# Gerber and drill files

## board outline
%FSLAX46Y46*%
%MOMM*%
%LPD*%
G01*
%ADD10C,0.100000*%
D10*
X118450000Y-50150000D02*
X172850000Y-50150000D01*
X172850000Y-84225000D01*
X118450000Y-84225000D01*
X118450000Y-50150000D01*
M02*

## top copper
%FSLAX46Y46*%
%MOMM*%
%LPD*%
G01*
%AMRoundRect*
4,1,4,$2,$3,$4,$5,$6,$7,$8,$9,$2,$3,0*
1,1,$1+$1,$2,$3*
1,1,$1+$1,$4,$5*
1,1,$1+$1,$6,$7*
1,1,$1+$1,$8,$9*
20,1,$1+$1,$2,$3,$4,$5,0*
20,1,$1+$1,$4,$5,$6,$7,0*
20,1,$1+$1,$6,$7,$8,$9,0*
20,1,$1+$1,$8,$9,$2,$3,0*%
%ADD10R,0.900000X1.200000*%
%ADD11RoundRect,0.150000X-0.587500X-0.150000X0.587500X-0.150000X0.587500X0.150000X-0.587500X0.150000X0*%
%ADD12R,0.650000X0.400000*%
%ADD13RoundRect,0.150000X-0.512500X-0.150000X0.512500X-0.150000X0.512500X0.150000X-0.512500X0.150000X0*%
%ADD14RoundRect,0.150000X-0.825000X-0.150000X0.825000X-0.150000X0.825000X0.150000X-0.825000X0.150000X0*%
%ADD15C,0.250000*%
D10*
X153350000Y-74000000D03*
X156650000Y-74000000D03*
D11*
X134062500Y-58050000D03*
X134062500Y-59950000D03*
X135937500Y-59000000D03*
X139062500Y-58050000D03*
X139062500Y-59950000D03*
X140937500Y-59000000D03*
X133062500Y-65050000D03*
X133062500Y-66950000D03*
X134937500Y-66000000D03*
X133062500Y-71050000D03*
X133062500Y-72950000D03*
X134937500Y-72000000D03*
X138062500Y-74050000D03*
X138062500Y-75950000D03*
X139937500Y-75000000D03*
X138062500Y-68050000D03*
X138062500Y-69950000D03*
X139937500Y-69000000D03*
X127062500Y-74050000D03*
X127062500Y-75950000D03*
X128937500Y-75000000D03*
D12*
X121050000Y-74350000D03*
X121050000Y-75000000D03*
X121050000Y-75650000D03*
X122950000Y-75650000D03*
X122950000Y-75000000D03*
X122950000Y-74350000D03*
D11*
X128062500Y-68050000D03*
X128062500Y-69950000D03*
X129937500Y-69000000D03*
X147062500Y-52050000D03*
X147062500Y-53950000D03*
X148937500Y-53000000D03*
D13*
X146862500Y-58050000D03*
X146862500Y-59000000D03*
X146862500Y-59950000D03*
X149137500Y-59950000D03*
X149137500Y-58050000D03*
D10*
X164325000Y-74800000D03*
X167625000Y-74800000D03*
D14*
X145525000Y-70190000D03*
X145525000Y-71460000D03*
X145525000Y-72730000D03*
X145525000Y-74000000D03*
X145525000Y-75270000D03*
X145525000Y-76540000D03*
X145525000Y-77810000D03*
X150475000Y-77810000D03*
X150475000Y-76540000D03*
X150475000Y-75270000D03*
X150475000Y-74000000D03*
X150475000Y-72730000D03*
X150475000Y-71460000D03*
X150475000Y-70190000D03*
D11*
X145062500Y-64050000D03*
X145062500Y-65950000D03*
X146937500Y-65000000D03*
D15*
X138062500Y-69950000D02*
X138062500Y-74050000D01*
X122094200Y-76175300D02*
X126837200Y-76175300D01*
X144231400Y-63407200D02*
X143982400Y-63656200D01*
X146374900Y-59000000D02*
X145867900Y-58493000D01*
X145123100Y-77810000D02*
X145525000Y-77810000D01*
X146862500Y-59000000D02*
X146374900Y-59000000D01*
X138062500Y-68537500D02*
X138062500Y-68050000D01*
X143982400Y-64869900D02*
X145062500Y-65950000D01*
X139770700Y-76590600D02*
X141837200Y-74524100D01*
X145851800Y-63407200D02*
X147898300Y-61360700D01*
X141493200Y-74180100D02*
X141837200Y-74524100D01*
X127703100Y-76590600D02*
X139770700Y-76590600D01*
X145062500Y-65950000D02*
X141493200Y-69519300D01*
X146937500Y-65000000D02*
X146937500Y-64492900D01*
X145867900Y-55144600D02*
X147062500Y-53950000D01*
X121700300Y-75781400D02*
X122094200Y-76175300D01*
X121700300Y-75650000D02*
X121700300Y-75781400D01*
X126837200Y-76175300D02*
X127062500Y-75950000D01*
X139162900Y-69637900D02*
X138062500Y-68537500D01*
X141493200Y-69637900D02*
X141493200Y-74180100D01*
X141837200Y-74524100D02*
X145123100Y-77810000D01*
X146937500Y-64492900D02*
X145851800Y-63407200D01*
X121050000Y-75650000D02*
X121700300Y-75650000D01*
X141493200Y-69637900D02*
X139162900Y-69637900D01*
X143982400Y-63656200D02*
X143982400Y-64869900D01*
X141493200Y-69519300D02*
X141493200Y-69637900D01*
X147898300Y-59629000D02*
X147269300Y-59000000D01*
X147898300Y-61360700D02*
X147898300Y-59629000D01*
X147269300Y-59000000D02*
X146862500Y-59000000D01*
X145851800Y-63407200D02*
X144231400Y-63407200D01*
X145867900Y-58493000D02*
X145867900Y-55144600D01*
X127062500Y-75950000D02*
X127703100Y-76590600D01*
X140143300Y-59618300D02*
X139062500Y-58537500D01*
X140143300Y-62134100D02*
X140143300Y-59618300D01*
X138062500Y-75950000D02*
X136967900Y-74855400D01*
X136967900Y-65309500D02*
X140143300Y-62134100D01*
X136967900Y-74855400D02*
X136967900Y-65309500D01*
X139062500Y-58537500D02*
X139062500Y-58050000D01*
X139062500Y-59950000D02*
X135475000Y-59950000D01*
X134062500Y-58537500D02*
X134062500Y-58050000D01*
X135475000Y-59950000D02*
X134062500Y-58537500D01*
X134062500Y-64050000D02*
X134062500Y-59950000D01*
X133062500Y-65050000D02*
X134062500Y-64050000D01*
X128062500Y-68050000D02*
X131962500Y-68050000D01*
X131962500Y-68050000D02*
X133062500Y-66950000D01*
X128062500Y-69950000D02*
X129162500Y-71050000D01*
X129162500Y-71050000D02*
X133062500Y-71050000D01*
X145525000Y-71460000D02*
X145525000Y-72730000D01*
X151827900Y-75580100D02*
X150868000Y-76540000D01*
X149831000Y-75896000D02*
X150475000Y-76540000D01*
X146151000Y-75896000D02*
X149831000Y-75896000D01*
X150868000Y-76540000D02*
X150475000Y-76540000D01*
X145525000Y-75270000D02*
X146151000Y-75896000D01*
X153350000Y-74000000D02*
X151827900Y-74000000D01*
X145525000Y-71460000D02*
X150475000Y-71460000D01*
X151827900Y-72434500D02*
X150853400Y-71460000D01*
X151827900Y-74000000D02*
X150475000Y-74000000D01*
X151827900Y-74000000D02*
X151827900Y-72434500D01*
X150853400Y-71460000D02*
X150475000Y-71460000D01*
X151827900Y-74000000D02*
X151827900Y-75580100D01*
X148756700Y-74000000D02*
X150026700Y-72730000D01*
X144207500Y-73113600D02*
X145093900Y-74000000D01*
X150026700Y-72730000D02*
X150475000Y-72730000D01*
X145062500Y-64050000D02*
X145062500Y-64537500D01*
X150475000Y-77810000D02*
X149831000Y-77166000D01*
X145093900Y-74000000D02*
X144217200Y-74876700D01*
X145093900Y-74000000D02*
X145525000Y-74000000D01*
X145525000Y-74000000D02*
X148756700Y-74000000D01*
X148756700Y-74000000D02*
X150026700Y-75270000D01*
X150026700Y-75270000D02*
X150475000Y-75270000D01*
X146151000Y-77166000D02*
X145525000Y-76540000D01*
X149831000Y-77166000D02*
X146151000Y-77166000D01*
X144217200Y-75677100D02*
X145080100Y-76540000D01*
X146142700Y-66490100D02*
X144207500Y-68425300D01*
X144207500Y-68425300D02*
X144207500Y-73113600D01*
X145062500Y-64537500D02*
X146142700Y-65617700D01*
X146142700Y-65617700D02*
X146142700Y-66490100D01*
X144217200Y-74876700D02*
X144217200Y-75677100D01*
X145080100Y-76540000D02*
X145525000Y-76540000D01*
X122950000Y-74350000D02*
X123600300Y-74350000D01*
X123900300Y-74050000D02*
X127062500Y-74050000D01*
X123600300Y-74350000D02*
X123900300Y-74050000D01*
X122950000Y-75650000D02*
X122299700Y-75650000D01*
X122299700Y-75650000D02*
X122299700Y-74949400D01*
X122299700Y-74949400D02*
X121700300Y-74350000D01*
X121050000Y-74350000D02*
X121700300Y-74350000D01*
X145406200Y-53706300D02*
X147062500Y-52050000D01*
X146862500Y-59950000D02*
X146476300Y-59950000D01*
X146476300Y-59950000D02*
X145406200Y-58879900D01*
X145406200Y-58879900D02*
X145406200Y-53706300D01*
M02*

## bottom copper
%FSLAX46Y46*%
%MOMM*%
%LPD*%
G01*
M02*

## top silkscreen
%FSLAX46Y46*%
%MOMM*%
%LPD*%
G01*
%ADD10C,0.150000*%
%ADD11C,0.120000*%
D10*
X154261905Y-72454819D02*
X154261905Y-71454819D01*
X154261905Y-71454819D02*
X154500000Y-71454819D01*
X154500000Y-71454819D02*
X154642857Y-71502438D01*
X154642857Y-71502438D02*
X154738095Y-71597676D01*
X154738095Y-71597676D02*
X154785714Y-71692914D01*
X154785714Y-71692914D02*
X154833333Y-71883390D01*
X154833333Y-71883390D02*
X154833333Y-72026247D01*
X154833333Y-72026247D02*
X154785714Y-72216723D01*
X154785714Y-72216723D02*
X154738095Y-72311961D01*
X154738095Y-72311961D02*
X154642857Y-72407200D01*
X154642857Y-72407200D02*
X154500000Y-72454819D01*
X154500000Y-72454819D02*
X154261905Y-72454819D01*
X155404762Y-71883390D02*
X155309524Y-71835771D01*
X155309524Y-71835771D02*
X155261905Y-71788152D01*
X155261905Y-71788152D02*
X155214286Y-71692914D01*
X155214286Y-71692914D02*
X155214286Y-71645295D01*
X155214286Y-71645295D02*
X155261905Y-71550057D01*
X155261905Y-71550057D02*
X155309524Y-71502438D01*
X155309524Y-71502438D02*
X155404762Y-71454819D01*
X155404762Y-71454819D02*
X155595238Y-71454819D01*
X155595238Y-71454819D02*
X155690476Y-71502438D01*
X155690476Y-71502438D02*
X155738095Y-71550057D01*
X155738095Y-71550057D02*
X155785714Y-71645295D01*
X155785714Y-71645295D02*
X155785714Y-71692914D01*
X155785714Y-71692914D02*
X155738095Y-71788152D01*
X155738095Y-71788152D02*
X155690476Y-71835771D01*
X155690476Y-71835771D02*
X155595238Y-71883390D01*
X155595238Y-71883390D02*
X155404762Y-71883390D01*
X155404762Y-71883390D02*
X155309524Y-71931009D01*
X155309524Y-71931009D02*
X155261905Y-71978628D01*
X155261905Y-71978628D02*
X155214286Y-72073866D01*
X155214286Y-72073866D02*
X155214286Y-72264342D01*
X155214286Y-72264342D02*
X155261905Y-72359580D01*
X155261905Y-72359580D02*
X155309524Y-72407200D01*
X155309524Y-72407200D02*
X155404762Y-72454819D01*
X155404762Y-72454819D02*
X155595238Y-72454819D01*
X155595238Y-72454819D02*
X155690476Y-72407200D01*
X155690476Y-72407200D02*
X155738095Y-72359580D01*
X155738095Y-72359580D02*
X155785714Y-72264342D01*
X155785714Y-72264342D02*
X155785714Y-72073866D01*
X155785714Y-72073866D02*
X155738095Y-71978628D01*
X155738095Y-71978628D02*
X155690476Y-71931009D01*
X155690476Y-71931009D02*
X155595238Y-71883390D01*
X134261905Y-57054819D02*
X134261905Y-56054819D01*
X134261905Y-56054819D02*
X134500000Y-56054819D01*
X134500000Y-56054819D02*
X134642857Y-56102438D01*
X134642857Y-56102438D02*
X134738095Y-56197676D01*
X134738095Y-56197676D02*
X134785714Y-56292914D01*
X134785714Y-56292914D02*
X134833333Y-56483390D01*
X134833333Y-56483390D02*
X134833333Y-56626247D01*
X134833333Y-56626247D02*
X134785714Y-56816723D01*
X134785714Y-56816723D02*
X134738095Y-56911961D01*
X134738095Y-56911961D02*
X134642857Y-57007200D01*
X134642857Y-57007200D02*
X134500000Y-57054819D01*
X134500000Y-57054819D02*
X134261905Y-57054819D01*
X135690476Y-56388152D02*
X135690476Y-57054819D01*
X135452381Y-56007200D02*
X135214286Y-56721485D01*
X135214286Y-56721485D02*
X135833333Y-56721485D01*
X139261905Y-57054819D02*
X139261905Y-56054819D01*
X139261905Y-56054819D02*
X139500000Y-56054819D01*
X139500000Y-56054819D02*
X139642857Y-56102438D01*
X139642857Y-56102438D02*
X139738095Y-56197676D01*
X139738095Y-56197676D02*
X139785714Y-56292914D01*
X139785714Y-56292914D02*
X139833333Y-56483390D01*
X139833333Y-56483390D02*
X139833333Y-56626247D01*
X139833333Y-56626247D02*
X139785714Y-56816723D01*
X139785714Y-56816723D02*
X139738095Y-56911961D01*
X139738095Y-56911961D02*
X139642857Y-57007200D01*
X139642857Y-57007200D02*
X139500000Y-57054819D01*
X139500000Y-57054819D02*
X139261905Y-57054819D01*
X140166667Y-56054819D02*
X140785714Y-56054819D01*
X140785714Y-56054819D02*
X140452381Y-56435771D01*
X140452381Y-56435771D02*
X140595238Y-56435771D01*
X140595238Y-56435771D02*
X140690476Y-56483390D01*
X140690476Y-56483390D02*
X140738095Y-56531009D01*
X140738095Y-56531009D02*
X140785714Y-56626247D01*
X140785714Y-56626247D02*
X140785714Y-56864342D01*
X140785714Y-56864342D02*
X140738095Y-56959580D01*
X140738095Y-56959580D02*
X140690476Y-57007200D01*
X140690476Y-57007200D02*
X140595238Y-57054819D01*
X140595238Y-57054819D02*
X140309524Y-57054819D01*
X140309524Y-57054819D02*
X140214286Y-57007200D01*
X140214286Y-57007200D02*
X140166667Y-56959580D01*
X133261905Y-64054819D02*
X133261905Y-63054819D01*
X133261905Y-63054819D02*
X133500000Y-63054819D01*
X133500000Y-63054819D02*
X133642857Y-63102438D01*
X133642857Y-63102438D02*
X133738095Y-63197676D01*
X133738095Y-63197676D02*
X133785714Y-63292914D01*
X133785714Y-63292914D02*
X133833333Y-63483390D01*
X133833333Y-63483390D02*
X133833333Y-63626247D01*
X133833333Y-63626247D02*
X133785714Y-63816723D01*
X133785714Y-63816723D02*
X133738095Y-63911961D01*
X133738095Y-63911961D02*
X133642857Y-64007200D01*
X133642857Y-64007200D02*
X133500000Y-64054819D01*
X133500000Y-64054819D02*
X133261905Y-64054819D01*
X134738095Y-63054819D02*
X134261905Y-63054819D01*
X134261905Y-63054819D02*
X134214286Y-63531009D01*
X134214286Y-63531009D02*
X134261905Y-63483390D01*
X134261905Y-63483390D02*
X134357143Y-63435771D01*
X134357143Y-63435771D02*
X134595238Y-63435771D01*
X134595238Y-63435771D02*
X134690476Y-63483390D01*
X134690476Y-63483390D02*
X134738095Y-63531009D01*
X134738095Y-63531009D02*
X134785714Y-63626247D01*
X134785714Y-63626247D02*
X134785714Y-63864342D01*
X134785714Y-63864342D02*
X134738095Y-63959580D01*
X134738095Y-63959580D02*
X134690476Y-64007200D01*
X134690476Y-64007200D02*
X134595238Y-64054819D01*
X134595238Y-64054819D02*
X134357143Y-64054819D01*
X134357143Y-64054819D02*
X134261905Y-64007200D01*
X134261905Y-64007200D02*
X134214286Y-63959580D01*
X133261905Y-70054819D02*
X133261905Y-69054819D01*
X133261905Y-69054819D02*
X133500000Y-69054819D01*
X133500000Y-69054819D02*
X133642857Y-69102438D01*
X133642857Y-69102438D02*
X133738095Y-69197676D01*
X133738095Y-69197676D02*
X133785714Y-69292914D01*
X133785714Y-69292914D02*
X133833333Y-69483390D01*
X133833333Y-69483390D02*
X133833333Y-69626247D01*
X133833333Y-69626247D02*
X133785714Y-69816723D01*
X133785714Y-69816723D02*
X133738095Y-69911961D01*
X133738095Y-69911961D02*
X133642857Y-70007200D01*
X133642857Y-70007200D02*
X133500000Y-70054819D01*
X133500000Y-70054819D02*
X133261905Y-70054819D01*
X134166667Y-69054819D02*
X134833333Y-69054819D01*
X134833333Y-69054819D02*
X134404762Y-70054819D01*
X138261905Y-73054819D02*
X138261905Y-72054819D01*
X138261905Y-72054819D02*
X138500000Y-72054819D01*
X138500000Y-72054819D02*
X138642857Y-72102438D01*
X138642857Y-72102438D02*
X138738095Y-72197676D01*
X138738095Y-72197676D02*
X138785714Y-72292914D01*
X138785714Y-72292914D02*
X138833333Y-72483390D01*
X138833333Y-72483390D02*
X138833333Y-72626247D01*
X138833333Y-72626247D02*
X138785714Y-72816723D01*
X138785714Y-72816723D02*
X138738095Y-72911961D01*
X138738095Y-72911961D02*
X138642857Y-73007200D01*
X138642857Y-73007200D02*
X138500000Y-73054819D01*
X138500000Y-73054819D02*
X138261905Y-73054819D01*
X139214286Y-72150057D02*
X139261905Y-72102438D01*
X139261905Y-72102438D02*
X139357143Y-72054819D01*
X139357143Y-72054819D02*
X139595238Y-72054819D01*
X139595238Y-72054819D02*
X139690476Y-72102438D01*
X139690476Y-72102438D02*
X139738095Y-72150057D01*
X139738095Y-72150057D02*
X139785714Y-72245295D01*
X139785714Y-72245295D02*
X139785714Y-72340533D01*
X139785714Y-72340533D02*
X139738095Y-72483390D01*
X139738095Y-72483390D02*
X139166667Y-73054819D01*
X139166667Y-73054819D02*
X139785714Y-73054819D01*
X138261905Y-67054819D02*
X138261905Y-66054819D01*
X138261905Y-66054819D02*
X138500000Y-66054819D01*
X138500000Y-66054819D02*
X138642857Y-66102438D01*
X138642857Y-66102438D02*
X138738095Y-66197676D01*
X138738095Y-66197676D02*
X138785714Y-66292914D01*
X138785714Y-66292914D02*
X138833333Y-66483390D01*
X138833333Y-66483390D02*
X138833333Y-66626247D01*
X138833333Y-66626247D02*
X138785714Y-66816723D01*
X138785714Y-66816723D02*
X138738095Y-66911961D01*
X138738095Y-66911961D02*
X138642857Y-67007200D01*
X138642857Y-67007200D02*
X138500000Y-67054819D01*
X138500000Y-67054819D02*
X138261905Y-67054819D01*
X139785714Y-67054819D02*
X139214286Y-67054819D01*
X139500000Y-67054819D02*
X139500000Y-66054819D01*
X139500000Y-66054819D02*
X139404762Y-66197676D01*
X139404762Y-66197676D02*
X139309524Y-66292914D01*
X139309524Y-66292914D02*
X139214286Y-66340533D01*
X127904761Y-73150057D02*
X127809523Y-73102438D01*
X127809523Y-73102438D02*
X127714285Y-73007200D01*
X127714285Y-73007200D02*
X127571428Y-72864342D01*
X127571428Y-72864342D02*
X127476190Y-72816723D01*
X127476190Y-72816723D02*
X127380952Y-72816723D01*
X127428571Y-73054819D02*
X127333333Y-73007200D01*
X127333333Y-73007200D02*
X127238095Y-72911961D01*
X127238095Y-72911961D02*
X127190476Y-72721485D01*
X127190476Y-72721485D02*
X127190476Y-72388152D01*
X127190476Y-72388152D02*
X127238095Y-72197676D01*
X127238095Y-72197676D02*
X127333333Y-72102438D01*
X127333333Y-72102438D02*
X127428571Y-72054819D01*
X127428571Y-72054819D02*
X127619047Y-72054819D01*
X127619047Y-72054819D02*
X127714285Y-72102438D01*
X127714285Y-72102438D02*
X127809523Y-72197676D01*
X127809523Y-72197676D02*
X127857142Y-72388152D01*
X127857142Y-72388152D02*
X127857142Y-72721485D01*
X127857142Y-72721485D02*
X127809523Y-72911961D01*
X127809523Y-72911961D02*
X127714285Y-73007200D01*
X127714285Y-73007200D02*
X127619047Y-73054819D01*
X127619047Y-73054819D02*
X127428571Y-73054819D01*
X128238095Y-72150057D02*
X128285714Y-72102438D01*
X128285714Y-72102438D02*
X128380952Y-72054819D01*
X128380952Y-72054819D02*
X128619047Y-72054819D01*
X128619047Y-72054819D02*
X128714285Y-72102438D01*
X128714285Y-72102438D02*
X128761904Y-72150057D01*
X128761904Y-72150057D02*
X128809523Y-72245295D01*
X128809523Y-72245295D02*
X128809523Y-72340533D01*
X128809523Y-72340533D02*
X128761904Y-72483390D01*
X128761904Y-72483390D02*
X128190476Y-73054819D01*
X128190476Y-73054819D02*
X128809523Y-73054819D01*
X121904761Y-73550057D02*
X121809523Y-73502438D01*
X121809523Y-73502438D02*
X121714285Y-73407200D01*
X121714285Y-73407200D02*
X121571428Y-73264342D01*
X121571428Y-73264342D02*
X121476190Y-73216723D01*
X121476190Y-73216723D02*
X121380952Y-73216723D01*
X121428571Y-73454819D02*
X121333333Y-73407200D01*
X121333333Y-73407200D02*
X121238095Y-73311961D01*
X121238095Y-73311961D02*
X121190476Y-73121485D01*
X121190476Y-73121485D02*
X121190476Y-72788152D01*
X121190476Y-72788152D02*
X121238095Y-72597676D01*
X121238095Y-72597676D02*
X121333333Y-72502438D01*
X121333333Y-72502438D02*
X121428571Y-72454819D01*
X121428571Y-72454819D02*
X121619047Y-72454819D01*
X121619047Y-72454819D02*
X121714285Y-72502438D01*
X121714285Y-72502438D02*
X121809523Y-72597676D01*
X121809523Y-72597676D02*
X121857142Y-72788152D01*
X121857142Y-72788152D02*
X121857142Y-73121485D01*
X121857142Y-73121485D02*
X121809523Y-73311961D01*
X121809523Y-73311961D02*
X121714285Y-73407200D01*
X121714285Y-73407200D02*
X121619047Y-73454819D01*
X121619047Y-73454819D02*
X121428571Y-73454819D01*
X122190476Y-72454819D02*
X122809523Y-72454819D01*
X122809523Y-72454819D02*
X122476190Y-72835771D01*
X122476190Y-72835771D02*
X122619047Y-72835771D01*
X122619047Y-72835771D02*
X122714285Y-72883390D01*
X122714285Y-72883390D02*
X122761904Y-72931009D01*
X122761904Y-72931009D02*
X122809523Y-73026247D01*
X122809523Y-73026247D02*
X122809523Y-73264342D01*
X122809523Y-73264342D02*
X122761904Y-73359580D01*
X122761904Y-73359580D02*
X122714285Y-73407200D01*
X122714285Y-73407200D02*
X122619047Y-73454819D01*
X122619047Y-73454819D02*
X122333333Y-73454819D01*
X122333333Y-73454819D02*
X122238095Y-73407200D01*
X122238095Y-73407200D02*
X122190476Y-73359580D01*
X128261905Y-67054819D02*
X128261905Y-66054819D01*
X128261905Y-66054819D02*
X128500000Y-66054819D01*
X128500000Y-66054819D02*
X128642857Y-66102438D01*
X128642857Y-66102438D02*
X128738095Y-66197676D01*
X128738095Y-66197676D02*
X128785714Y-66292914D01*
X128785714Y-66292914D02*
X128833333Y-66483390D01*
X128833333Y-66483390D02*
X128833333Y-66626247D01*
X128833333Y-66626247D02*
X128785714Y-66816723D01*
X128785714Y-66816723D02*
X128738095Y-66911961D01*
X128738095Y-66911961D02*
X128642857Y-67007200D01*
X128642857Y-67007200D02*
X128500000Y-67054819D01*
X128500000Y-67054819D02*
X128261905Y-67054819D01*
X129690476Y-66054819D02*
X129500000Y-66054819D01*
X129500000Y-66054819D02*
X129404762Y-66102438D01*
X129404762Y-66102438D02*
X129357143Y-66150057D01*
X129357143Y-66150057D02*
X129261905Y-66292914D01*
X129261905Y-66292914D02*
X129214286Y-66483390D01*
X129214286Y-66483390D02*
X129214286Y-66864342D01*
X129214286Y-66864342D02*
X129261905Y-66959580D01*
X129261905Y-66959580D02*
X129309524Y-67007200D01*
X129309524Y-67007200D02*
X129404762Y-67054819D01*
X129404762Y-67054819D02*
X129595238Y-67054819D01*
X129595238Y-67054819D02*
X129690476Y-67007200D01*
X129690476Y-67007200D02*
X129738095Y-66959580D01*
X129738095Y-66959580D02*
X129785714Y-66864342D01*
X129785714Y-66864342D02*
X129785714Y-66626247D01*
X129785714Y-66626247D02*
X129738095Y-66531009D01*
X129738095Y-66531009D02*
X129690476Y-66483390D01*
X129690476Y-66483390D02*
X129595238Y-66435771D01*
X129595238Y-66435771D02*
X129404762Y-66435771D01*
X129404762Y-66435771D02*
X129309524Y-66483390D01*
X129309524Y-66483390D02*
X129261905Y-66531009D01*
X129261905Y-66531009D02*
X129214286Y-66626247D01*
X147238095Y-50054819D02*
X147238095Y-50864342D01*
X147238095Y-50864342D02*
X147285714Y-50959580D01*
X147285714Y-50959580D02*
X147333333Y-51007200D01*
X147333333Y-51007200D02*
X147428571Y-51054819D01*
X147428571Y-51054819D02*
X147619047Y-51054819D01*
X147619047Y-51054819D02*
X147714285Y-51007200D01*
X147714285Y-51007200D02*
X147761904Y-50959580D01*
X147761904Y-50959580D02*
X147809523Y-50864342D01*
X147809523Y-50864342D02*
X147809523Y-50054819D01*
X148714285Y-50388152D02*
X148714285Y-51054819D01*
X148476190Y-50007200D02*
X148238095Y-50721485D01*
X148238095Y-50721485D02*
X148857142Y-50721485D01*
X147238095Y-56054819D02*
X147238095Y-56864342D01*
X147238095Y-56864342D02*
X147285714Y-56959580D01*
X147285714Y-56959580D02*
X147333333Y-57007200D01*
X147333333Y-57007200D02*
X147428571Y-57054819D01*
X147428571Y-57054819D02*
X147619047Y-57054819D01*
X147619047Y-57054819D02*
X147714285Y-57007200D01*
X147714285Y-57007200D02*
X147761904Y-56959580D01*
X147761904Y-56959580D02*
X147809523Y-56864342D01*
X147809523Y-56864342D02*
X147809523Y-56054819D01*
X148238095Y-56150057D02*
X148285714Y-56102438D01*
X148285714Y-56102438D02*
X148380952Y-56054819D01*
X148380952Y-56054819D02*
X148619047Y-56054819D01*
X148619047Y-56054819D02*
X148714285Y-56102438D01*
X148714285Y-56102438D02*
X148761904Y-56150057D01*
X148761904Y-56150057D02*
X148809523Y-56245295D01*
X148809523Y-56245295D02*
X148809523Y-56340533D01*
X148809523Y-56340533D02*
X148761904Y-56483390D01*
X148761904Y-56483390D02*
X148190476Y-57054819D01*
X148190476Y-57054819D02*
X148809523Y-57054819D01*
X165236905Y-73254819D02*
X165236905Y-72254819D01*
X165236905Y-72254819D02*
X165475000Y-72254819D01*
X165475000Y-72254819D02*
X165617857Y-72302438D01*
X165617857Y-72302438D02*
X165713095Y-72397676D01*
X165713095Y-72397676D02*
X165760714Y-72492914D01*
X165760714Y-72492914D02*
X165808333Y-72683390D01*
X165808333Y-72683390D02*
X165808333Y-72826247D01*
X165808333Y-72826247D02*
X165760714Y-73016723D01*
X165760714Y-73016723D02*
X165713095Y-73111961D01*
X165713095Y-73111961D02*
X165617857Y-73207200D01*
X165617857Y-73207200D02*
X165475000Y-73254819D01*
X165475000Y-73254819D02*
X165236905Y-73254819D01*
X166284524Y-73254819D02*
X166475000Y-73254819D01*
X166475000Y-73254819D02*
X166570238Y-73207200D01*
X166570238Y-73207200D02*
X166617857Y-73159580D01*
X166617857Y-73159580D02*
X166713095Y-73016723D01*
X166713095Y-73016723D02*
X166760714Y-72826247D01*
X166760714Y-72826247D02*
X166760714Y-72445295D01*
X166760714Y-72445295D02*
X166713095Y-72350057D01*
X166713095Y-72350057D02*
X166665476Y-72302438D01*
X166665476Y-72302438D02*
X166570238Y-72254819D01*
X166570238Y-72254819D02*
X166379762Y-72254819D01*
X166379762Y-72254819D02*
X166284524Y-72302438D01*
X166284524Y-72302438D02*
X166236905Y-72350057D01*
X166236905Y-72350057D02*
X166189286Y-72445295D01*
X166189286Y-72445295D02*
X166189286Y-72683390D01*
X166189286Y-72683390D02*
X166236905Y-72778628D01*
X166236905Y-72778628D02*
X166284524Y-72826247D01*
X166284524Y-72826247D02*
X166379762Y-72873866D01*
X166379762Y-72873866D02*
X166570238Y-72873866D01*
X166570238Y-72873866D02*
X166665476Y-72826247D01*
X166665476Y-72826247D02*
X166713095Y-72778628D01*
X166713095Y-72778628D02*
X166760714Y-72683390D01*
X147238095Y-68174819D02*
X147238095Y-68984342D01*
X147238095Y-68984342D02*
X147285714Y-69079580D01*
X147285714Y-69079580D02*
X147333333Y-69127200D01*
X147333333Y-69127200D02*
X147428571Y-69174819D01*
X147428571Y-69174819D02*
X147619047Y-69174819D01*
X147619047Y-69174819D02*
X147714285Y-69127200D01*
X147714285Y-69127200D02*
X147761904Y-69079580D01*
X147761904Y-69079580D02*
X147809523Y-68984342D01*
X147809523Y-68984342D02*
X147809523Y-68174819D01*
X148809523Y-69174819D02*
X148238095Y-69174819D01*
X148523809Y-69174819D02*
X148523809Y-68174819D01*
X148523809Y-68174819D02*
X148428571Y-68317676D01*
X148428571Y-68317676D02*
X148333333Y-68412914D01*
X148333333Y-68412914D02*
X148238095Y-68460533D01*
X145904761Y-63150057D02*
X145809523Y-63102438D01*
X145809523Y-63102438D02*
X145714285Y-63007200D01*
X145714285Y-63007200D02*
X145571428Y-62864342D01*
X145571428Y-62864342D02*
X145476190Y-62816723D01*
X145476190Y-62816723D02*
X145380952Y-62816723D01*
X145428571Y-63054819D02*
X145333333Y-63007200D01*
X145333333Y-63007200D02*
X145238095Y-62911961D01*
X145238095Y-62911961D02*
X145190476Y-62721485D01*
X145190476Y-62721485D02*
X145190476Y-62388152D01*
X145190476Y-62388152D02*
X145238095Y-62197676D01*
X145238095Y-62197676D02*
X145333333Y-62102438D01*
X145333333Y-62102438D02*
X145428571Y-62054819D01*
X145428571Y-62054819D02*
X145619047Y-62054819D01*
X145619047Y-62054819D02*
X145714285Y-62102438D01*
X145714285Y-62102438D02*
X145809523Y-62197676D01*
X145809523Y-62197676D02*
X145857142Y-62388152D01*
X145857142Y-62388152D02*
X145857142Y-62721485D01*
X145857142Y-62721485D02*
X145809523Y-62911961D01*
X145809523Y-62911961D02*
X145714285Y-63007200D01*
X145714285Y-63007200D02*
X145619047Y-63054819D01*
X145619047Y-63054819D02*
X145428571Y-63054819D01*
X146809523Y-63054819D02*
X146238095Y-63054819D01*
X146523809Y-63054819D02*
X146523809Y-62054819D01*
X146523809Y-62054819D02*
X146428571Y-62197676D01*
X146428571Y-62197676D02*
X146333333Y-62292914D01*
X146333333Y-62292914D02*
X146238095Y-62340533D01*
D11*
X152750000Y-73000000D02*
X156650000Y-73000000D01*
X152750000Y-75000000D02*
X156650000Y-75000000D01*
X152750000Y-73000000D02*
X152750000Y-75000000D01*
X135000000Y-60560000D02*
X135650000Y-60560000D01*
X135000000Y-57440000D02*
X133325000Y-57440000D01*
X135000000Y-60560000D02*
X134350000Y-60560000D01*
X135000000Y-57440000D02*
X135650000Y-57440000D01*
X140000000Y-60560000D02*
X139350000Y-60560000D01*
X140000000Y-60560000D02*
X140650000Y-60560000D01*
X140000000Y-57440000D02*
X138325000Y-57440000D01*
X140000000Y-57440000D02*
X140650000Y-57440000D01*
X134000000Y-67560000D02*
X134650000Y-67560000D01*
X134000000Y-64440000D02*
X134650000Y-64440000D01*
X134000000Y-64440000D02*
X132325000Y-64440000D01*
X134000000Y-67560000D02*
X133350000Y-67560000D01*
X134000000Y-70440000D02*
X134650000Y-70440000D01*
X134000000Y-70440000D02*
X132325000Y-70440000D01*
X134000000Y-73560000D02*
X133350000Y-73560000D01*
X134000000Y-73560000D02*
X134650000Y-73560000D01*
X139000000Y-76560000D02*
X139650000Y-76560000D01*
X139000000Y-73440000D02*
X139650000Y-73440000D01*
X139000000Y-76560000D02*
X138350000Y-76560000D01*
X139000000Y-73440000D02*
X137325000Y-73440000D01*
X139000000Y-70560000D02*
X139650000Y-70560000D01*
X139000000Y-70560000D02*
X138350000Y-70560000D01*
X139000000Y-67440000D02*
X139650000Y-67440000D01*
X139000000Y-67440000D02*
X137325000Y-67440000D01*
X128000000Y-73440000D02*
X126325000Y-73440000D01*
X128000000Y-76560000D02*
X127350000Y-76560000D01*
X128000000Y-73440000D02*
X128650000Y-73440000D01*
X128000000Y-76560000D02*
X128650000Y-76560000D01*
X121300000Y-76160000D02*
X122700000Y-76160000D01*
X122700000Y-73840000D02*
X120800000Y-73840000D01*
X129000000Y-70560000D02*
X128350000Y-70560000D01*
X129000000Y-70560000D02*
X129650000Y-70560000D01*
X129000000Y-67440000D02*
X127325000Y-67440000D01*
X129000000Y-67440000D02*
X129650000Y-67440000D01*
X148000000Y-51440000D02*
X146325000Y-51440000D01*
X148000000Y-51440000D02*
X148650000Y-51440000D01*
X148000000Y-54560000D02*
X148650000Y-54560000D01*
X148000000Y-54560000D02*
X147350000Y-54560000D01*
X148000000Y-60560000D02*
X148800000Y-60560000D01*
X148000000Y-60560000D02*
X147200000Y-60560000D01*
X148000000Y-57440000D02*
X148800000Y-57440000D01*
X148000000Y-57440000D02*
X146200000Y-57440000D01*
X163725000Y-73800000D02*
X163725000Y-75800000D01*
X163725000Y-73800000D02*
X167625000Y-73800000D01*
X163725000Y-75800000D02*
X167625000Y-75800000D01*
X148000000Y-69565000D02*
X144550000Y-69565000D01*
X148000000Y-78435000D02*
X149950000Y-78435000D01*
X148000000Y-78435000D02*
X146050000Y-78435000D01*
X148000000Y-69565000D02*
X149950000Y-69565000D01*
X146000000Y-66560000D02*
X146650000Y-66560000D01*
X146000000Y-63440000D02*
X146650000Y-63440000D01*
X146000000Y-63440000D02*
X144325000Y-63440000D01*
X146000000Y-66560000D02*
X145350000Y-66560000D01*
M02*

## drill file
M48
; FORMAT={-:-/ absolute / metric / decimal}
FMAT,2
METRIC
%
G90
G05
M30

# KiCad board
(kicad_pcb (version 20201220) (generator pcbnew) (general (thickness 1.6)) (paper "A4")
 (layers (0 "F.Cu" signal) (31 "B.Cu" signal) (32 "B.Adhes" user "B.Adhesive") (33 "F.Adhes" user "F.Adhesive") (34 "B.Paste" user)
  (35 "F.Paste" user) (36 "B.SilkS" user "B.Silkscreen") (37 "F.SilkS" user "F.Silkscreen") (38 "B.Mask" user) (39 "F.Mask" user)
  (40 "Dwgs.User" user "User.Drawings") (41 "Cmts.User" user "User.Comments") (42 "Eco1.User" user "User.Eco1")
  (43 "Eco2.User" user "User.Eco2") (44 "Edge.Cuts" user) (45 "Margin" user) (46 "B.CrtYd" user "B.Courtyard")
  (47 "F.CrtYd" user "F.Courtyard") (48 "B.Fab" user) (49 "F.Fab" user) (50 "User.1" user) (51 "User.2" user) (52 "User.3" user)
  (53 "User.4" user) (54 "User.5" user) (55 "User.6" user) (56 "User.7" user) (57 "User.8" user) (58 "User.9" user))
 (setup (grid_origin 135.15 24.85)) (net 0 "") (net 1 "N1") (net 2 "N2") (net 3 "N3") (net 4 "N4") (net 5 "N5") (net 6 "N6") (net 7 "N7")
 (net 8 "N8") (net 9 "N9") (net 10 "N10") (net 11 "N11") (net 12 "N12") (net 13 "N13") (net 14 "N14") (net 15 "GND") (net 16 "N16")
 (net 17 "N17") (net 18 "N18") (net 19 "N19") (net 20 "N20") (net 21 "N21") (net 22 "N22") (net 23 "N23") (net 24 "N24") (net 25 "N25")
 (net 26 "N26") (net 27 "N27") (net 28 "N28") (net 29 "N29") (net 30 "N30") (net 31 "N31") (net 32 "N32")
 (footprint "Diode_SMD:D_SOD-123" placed (layer "F.Cu") (at 155 74)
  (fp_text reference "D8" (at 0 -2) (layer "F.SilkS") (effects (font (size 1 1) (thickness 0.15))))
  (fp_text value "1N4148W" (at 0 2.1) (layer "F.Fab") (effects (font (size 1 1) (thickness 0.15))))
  (fp_line (start -2.25 -1) (end 1.65 -1) (layer "F.SilkS") (width 0.12))
  (fp_line (start -2.25 1) (end 1.65 1) (layer "F.SilkS") (width 0.12))
  (fp_line (start -2.25 -1) (end -2.25 1) (layer "F.SilkS") (width 0.12))
  (pad "1" smd rect (at -1.65 0) (size 0.9 1.2) (layers "F.Cu" "F.Paste" "F.Mask") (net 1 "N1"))
  (pad "2" smd rect (at 1.65 0) (size 0.9 1.2) (layers "F.Cu" "F.Paste" "F.Mask") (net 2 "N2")))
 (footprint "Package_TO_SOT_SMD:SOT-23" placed (layer "F.Cu") (at 135 59)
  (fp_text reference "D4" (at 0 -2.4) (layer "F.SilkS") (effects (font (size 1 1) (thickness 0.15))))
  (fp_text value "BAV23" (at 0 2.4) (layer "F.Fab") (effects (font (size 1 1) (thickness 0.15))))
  (fp_line (start 0 1.56) (end 0.65 1.56) (layer "F.SilkS") (width 0.12))
  (fp_line (start 0 -1.56) (end -1.675 -1.56) (layer "F.SilkS") (width 0.12))
  (fp_line (start 0 1.56) (end -0.65 1.56) (layer "F.SilkS") (width 0.12))
  (fp_line (start 0 -1.56) (end 0.65 -1.56) (layer "F.SilkS") (width 0.12))
  (pad "1" smd roundrect (at -0.9375 -0.95) (size 1.475 0.6) (layers "F.Cu" "F.Paste" "F.Mask") (roundrect_rratio 0.25) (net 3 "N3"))
  (pad "2" smd roundrect (at -0.9375 0.95) (size 1.475 0.6) (layers "F.Cu" "F.Paste" "F.Mask") (roundrect_rratio 0.25) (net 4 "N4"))
  (pad "3" smd roundrect (at 0.9375 0) (size 1.475 0.6) (layers "F.Cu" "F.Paste" "F.Mask") (roundrect_rratio 0.25) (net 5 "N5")))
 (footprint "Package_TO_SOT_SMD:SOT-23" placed (layer "F.Cu") (at 140 59)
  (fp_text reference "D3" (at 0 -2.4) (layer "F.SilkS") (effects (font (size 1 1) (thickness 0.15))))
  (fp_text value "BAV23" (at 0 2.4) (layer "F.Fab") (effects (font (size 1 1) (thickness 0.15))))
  (fp_line (start 0 1.56) (end -0.65 1.56) (layer "F.SilkS") (width 0.12))
  (fp_line (start 0 1.56) (end 0.65 1.56) (layer "F.SilkS") (width 0.12))
  (fp_line (start 0 -1.56) (end -1.675 -1.56) (layer "F.SilkS") (width 0.12))
  (fp_line (start 0 -1.56) (end 0.65 -1.56) (layer "F.SilkS") (width 0.12))
  (pad "1" smd roundrect (at -0.9375 -0.95) (size 1.475 0.6) (layers "F.Cu" "F.Paste" "F.Mask") (roundrect_rratio 0.25) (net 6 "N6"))
  (pad "2" smd roundrect (at -0.9375 0.95) (size 1.475 0.6) (layers "F.Cu" "F.Paste" "F.Mask") (roundrect_rratio 0.25) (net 3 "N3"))
  (pad "3" smd roundrect (at 0.9375 0) (size 1.475 0.6) (layers "F.Cu" "F.Paste" "F.Mask") (roundrect_rratio 0.25) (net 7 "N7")))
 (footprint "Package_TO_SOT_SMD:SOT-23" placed (layer "F.Cu") (at 134 66)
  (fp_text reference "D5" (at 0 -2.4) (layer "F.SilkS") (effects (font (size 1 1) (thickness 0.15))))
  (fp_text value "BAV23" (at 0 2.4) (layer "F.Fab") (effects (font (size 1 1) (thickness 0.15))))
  (fp_line (start 0 1.56) (end 0.65 1.56) (layer "F.SilkS") (width 0.12))
  (fp_line (start 0 -1.56) (end 0.65 -1.56) (layer "F.SilkS") (width 0.12))
  (fp_line (start 0 -1.56) (end -1.675 -1.56) (layer "F.SilkS") (width 0.12))
  (fp_line (start 0 1.56) (end -0.65 1.56) (layer "F.SilkS") (width 0.12))
  (pad "1" smd roundrect (at -0.9375 -0.95) (size 1.475 0.6) (layers "F.Cu" "F.Paste" "F.Mask") (roundrect_rratio 0.25) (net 4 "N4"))
  (pad "2" smd roundrect (at -0.9375 0.95) (size 1.475 0.6) (layers "F.Cu" "F.Paste" "F.Mask") (roundrect_rratio 0.25) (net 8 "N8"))
  (pad "3" smd roundrect (at 0.9375 0) (size 1.475 0.6) (layers "F.Cu" "F.Paste" "F.Mask") (roundrect_rratio 0.25) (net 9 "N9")))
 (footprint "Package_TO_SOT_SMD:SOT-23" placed (layer "F.Cu") (at 134 72)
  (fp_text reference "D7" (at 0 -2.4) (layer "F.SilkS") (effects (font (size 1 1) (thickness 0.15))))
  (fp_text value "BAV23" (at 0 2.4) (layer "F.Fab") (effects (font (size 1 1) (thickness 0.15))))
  (fp_line (start 0 -1.56) (end 0.65 -1.56) (layer "F.SilkS") (width 0.12))
  (fp_line (start 0 -1.56) (end -1.675 -1.56) (layer "F.SilkS") (width 0.12))
  (fp_line (start 0 1.56) (end -0.65 1.56) (layer "F.SilkS") (width 0.12))
  (fp_line (start 0 1.56) (end 0.65 1.56) (layer "F.SilkS") (width 0.12))
  (pad "1" smd roundrect (at -0.9375 -0.95) (size 1.475 0.6) (layers "F.Cu" "F.Paste" "F.Mask") (roundrect_rratio 0.25) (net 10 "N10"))
  (pad "2" smd roundrect (at -0.9375 0.95) (size 1.475 0.6) (layers "F.Cu" "F.Paste" "F.Mask") (roundrect_rratio 0.25) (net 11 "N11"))
  (pad "3" smd roundrect (at 0.9375 0) (size 1.475 0.6) (layers "F.Cu" "F.Paste" "F.Mask") (roundrect_rratio 0.25) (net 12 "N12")))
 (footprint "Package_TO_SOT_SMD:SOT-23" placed (layer "F.Cu") (at 139 75)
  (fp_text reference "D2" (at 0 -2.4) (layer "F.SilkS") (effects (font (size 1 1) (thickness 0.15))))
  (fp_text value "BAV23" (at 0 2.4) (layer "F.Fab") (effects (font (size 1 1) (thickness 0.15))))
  (fp_line (start 0 1.56) (end 0.65 1.56) (layer "F.SilkS") (width 0.12))
  (fp_line (start 0 -1.56) (end 0.65 -1.56) (layer "F.SilkS") (width 0.12))
  (fp_line (start 0 1.56) (end -0.65 1.56) (layer "F.SilkS") (width 0.12))
  (fp_line (start 0 -1.56) (end -1.675 -1.56) (layer "F.SilkS") (width 0.12))
  (pad "1" smd roundrect (at -0.9375 -0.95) (size 1.475 0.6) (layers "F.Cu" "F.Paste" "F.Mask") (roundrect_rratio 0.25) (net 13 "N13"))
  (pad "2" smd roundrect (at -0.9375 0.95) (size 1.475 0.6) (layers "F.Cu" "F.Paste" "F.Mask") (roundrect_rratio 0.25) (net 6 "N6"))
  (pad "3" smd roundrect (at 0.9375 0) (size 1.475 0.6) (layers "F.Cu" "F.Paste" "F.Mask") (roundrect_rratio 0.25) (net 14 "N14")))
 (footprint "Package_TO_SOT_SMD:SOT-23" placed (layer "F.Cu") (at 139 69)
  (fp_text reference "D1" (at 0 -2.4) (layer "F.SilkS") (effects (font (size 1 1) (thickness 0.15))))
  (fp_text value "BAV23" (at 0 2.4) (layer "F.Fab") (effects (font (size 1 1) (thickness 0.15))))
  (fp_line (start 0 1.56) (end 0.65 1.56) (layer "F.SilkS") (width 0.12))
  (fp_line (start 0 1.56) (end -0.65 1.56) (layer "F.SilkS") (width 0.12))
  (fp_line (start 0 -1.56) (end 0.65 -1.56) (layer "F.SilkS") (width 0.12))
  (fp_line (start 0 -1.56) (end -1.675 -1.56) (layer "F.SilkS") (width 0.12))
  (pad "1" smd roundrect (at -0.9375 -0.95) (size 1.475 0.6) (layers "F.Cu" "F.Paste" "F.Mask") (roundrect_rratio 0.25) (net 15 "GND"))
  (pad "2" smd roundrect (at -0.9375 0.95) (size 1.475 0.6) (layers "F.Cu" "F.Paste" "F.Mask") (roundrect_rratio 0.25) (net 13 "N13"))
  (pad "3" smd roundrect (at 0.9375 0) (size 1.475 0.6) (layers "F.Cu" "F.Paste" "F.Mask") (roundrect_rratio 0.25) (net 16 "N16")))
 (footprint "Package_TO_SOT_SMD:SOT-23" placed (layer "F.Cu") (at 128 75)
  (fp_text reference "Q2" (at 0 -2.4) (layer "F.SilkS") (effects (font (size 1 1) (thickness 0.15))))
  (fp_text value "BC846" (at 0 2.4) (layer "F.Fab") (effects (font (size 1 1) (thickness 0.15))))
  (fp_line (start 0 -1.56) (end -1.675 -1.56) (layer "F.SilkS") (width 0.12))
  (fp_line (start 0 1.56) (end -0.65 1.56) (layer "F.SilkS") (width 0.12))
  (fp_line (start 0 -1.56) (end 0.65 -1.56) (layer "F.SilkS") (width 0.12))
  (fp_line (start 0 1.56) (end 0.65 1.56) (layer "F.SilkS") (width 0.12))
  (pad "1" smd roundrect (at -0.9375 -0.95) (size 1.475 0.6) (layers "F.Cu" "F.Paste" "F.Mask") (roundrect_rratio 0.25) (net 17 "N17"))
  (pad "2" smd roundrect (at -0.9375 0.95) (size 1.475 0.6) (layers "F.Cu" "F.Paste" "F.Mask") (roundrect_rratio 0.25) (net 15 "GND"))
  (pad "3" smd roundrect (at 0.9375 0) (size 1.475 0.6) (layers "F.Cu" "F.Paste" "F.Mask") (roundrect_rratio 0.25) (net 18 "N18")))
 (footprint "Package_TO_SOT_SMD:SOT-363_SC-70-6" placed (layer "F.Cu") (at 122 75)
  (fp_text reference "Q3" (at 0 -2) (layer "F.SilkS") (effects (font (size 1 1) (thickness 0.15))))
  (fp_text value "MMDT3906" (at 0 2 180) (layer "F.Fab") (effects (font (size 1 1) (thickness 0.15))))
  (fp_line (start -0.7 1.16) (end 0.7 1.16) (layer "F.SilkS") (width 0.12))
  (fp_line (start 0.7 -1.16) (end -1.2 -1.16) (layer "F.SilkS") (width 0.12))
  (pad "1" smd rect (at -0.95 -0.65) (size 0.65 0.4) (layers "F.Cu" "F.Paste" "F.Mask") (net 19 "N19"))
  (pad "2" smd rect (at -0.95 0) (size 0.65 0.4) (layers "F.Cu" "F.Paste" "F.Mask") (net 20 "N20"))
  (pad "3" smd rect (at -0.95 0.65) (size 0.65 0.4) (layers "F.Cu" "F.Paste" "F.Mask") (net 15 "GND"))
  (pad "4" smd rect (at 0.95 0.65) (size 0.65 0.4) (layers "F.Cu" "F.Paste" "F.Mask") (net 19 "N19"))
  (pad "5" smd rect (at 0.95 0) (size 0.65 0.4) (layers "F.Cu" "F.Paste" "F.Mask") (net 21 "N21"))
  (pad "6" smd rect (at 0.95 -0.65) (size 0.65 0.4) (layers "F.Cu" "F.Paste" "F.Mask") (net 17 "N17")))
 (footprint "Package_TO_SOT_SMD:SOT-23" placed (layer "F.Cu") (at 129 69)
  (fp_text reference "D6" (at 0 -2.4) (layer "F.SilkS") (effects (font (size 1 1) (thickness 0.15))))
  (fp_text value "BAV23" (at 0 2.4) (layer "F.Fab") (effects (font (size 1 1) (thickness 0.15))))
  (fp_line (start 0 1.56) (end -0.65 1.56) (layer "F.SilkS") (width 0.12))
  (fp_line (start 0 1.56) (end 0.65 1.56) (layer "F.SilkS") (width 0.12))
  (fp_line (start 0 -1.56) (end -1.675 -1.56) (layer "F.SilkS") (width 0.12))
  (fp_line (start 0 -1.56) (end 0.65 -1.56) (layer "F.SilkS") (width 0.12))
  (pad "1" smd roundrect (at -0.9375 -0.95) (size 1.475 0.6) (layers "F.Cu" "F.Paste" "F.Mask") (roundrect_rratio 0.25) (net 8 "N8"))
  (pad "2" smd roundrect (at -0.9375 0.95) (size 1.475 0.6) (layers "F.Cu" "F.Paste" "F.Mask") (roundrect_rratio 0.25) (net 10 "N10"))
  (pad "3" smd roundrect (at 0.9375 0) (size 1.475 0.6) (layers "F.Cu" "F.Paste" "F.Mask") (roundrect_rratio 0.25) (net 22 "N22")))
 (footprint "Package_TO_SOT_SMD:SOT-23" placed (layer "F.Cu") (at 148 53)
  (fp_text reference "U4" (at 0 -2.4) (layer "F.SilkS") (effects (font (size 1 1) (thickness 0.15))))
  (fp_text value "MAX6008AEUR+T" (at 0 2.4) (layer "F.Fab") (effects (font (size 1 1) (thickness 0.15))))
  (fp_line (start 0 -1.56) (end -1.675 -1.56) (layer "F.SilkS") (width 0.12))
  (fp_line (start 0 -1.56) (end 0.65 -1.56) (layer "F.SilkS") (width 0.12))
  (fp_line (start 0 1.56) (end 0.65 1.56) (layer "F.SilkS") (width 0.12))
  (fp_line (start 0 1.56) (end -0.65 1.56) (layer "F.SilkS") (width 0.12))
  (pad "1" smd roundrect (at -0.9375 -0.95) (size 1.475 0.6) (layers "F.Cu" "F.Paste" "F.Mask") (roundrect_rratio 0.25) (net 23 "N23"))
  (pad "2" smd roundrect (at -0.9375 0.95) (size 1.475 0.6) (layers "F.Cu" "F.Paste" "F.Mask") (roundrect_rratio 0.25) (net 15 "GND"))
  (pad "3" smd roundrect (at 0.9375 0) (size 1.475 0.6) (layers "F.Cu" "F.Paste" "F.Mask") (roundrect_rratio 0.25) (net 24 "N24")))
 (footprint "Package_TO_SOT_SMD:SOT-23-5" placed (layer "F.Cu") (at 148 59)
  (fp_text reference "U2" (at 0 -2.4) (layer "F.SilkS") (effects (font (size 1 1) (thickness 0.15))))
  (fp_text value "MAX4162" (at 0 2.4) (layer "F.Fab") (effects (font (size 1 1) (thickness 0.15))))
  (fp_line (start 0 1.56) (end 0.8 1.56) (layer "F.SilkS") (width 0.12))
  (fp_line (start 0 1.56) (end -0.8 1.56) (layer "F.SilkS") (width 0.12))
  (fp_line (start 0 -1.56) (end 0.8 -1.56) (layer "F.SilkS") (width 0.12))
  (fp_line (start 0 -1.56) (end -1.8 -1.56) (layer "F.SilkS") (width 0.12))
  (pad "1" smd roundrect (at -1.1375 -0.95) (size 1.325 0.6) (layers "F.Cu" "F.Paste" "F.Mask") (roundrect_rratio 0.25) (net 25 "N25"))
  (pad "2" smd roundrect (at -1.1375 0) (size 1.325 0.6) (layers "F.Cu" "F.Paste" "F.Mask") (roundrect_rratio 0.25) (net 15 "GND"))
  (pad "3" smd roundrect (at -1.1375 0.95) (size 1.325 0.6) (layers "F.Cu" "F.Paste" "F.Mask") (roundrect_rratio 0.25) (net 23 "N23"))
  (pad "4" smd roundrect (at 1.1375 0.95) (size 1.325 0.6) (layers "F.Cu" "F.Paste" "F.Mask") (roundrect_rratio 0.25) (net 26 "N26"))
  (pad "5" smd roundrect (at 1.1375 -0.95) (size 1.325 0.6) (layers "F.Cu" "F.Paste" "F.Mask") (roundrect_rratio 0.25) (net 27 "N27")))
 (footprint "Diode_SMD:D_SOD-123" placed (layer "F.Cu") (at 165.975 74.8)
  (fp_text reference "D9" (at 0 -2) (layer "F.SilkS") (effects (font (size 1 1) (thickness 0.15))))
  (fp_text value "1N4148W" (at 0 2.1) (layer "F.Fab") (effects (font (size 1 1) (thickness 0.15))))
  (fp_line (start -2.25 -1) (end -2.25 1) (layer "F.SilkS") (width 0.12))
  (fp_line (start -2.25 -1) (end 1.65 -1) (layer "F.SilkS") (width 0.12))
  (fp_line (start -2.25 1) (end 1.65 1) (layer "F.SilkS") (width 0.12))
  (pad "1" smd rect (at -1.65 0) (size 0.9 1.2) (layers "F.Cu" "F.Paste" "F.Mask") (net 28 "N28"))
  (pad "2" smd rect (at 1.65 0) (size 0.9 1.2) (layers "F.Cu" "F.Paste" "F.Mask") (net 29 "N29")))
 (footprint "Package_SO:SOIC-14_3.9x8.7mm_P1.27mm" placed (layer "F.Cu") (at 148 74)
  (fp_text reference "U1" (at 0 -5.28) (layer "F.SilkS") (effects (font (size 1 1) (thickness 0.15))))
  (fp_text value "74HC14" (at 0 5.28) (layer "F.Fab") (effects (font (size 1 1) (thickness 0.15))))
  (fp_line (start 0 -4.435) (end -3.45 -4.435) (layer "F.SilkS") (width 0.12))
  (fp_line (start 0 4.435) (end 1.95 4.435) (layer "F.SilkS") (width 0.12))
  (fp_line (start 0 4.435) (end -1.95 4.435) (layer "F.SilkS") (width 0.12))
  (fp_line (start 0 -4.435) (end 1.95 -4.435) (layer "F.SilkS") (width 0.12))
  (pad "1" smd roundrect (at -2.475 -3.81) (size 1.95 0.6) (layers "F.Cu" "F.Paste" "F.Mask") (roundrect_rratio 0.25) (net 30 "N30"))
  (pad "2" smd roundrect (at -2.475 -2.54) (size 1.95 0.6) (layers "F.Cu" "F.Paste" "F.Mask") (roundrect_rratio 0.25) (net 1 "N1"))
  (pad "3" smd roundrect (at -2.475 -1.27) (size 1.95 0.6) (layers "F.Cu" "F.Paste" "F.Mask") (roundrect_rratio 0.25) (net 1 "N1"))
  (pad "4" smd roundrect (at -2.475 0) (size 1.95 0.6) (layers "F.Cu" "F.Paste" "F.Mask") (roundrect_rratio 0.25) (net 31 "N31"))
  (pad "5" smd roundrect (at -2.475 1.27) (size 1.95 0.6) (layers "F.Cu" "F.Paste" "F.Mask") (roundrect_rratio 0.25) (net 1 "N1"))
  (pad "6" smd roundrect (at -2.475 2.54) (size 1.95 0.6) (layers "F.Cu" "F.Paste" "F.Mask") (roundrect_rratio 0.25) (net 31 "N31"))
  (pad "7" smd roundrect (at -2.475 3.81) (size 1.95 0.6) (layers "F.Cu" "F.Paste" "F.Mask") (roundrect_rratio 0.25) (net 15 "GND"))
  (pad "8" smd roundrect (at 2.475 3.81) (size 1.95 0.6) (layers "F.Cu" "F.Paste" "F.Mask") (roundrect_rratio 0.25) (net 31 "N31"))
  (pad "9" smd roundrect (at 2.475 2.54) (size 1.95 0.6) (layers "F.Cu" "F.Paste" "F.Mask") (roundrect_rratio 0.25) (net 1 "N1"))
  (pad "10" smd roundrect (at 2.475 1.27) (size 1.95 0.6) (layers "F.Cu" "F.Paste" "F.Mask") (roundrect_rratio 0.25) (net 31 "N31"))
  (pad "11" smd roundrect (at 2.475 0) (size 1.95 0.6) (layers "F.Cu" "F.Paste" "F.Mask") (roundrect_rratio 0.25) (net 1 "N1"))
  (pad "12" smd roundrect (at 2.475 -1.27) (size 1.95 0.6) (layers "F.Cu" "F.Paste" "F.Mask") (roundrect_rratio 0.25) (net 31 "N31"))
  (pad "13" smd roundrect (at 2.475 -2.54) (size 1.95 0.6) (layers "F.Cu" "F.Paste" "F.Mask") (roundrect_rratio 0.25) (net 1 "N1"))
  (pad "14" smd roundrect (at 2.475 -3.81) (size 1.95 0.6) (layers "F.Cu" "F.Paste" "F.Mask") (roundrect_rratio 0.25) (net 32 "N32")))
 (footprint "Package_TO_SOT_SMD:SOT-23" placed (layer "F.Cu") (at 146 65)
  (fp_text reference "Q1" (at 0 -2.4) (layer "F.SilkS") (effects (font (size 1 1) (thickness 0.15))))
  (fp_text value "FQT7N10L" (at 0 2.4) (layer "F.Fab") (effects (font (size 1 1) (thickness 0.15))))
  (fp_line (start 0 1.56) (end 0.65 1.56) (layer "F.SilkS") (width 0.12))
  (fp_line (start 0 -1.56) (end 0.65 -1.56) (layer "F.SilkS") (width 0.12))
  (fp_line (start 0 -1.56) (end -1.675 -1.56) (layer "F.SilkS") (width 0.12))
  (fp_line (start 0 1.56) (end -0.65 1.56) (layer "F.SilkS") (width 0.12))
  (pad "1" smd roundrect (at -0.9375 -0.95) (size 1.475 0.6) (layers "F.Cu" "F.Paste" "F.Mask") (roundrect_rratio 0.25) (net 31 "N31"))
  (pad "2" smd roundrect (at -0.9375 0.95) (size 1.475 0.6) (layers "F.Cu" "F.Paste" "F.Mask") (roundrect_rratio 0.25) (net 15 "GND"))
  (pad "3" smd roundrect (at 0.9375 0) (size 1.475 0.6) (layers "F.Cu" "F.Paste" "F.Mask") (roundrect_rratio 0.25) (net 15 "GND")))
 (gr_rect (start 118.45 50.15) (end 172.85 84.225) (layer "Edge.Cuts") (width 0.1) (fill none))
 (segment (start 138.0625 69.95) (end 138.0625 74.05) (width 0.25) (layer "F.Cu") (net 13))
 (segment (start 122.0942 76.1753) (end 126.8372 76.1753) (width 0.25) (layer "F.Cu") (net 15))
 (segment (start 144.2314 63.4072) (end 143.9824 63.6562) (width 0.25) (layer "F.Cu") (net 15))
 (segment (start 146.3749 59) (end 145.8679 58.493) (width 0.25) (layer "F.Cu") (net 15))
 (segment (start 145.1231 77.81) (end 145.525 77.81) (width 0.25) (layer "F.Cu") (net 15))
 (segment (start 146.8625 59) (end 146.3749 59) (width 0.25) (layer "F.Cu") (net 15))
 (segment (start 138.0625 68.5375) (end 138.0625 68.05) (width 0.25) (layer "F.Cu") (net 15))
 (segment (start 143.9824 64.8699) (end 145.0625 65.95) (width 0.25) (layer "F.Cu") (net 15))
 (segment (start 139.7707 76.5906) (end 141.8372 74.5241) (width 0.25) (layer "F.Cu") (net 15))
 (segment (start 145.8518 63.4072) (end 147.8983 61.3607) (width 0.25) (layer "F.Cu") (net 15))
 (segment (start 141.4932 74.1801) (end 141.8372 74.5241) (width 0.25) (layer "F.Cu") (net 15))
 (segment (start 127.7031 76.5906) (end 139.7707 76.5906) (width 0.25) (layer "F.Cu") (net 15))
 (segment (start 145.0625 65.95) (end 141.4932 69.5193) (width 0.25) (layer "F.Cu") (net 15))
 (segment (start 146.9375 65) (end 146.9375 64.4929) (width 0.25) (layer "F.Cu") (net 15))
 (segment (start 145.8679 55.1446) (end 147.0625 53.95) (width 0.25) (layer "F.Cu") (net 15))
 (segment (start 121.7003 75.7814) (end 122.0942 76.1753) (width 0.25) (layer "F.Cu") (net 15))
 (segment (start 121.7003 75.65) (end 121.7003 75.7814) (width 0.25) (layer "F.Cu") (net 15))
 (segment (start 126.8372 76.1753) (end 127.0625 75.95) (width 0.25) (layer "F.Cu") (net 15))
 (segment (start 139.1629 69.6379) (end 138.0625 68.5375) (width 0.25) (layer "F.Cu") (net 15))
 (segment (start 141.4932 69.6379) (end 141.4932 74.1801) (width 0.25) (layer "F.Cu") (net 15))
 (segment (start 141.8372 74.5241) (end 145.1231 77.81) (width 0.25) (layer "F.Cu") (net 15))
 (segment (start 146.9375 64.4929) (end 145.8518 63.4072) (width 0.25) (layer "F.Cu") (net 15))
 (segment (start 121.05 75.65) (end 121.7003 75.65) (width 0.25) (layer "F.Cu") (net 15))
 (segment (start 141.4932 69.6379) (end 139.1629 69.6379) (width 0.25) (layer "F.Cu") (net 15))
 (segment (start 143.9824 63.6562) (end 143.9824 64.8699) (width 0.25) (layer "F.Cu") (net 15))
 (segment (start 141.4932 69.5193) (end 141.4932 69.6379) (width 0.25) (layer "F.Cu") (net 15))
 (segment (start 147.8983 59.629) (end 147.2693 59) (width 0.25) (layer "F.Cu") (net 15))
 (segment (start 147.8983 61.3607) (end 147.8983 59.629) (width 0.25) (layer "F.Cu") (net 15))
 (segment (start 147.2693 59) (end 146.8625 59) (width 0.25) (layer "F.Cu") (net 15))
 (segment (start 145.8518 63.4072) (end 144.2314 63.4072) (width 0.25) (layer "F.Cu") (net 15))
 (segment (start 145.8679 58.493) (end 145.8679 55.1446) (width 0.25) (layer "F.Cu") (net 15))
 (segment (start 127.0625 75.95) (end 127.7031 76.5906) (width 0.25) (layer "F.Cu") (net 15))
 (segment (start 140.1433 59.6183) (end 139.0625 58.5375) (width 0.25) (layer "F.Cu") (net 6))
 (segment (start 140.1433 62.1341) (end 140.1433 59.6183) (width 0.25) (layer "F.Cu") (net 6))
 (segment (start 138.0625 75.95) (end 136.9679 74.8554) (width 0.25) (layer "F.Cu") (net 6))
 (segment (start 136.9679 65.3095) (end 140.1433 62.1341) (width 0.25) (layer "F.Cu") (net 6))
 (segment (start 136.9679 74.8554) (end 136.9679 65.3095) (width 0.25) (layer "F.Cu") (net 6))
 (segment (start 139.0625 58.5375) (end 139.0625 58.05) (width 0.25) (layer "F.Cu") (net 6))
 (segment (start 139.0625 59.95) (end 135.475 59.95) (width 0.25) (layer "F.Cu") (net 3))
 (segment (start 134.0625 58.5375) (end 134.0625 58.05) (width 0.25) (layer "F.Cu") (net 3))
 (segment (start 135.475 59.95) (end 134.0625 58.5375) (width 0.25) (layer "F.Cu") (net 3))
 (segment (start 134.0625 64.05) (end 134.0625 59.95) (width 0.25) (layer "F.Cu") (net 4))
 (segment (start 133.0625 65.05) (end 134.0625 64.05) (width 0.25) (layer "F.Cu") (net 4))
 (segment (start 128.0625 68.05) (end 131.9625 68.05) (width 0.25) (layer "F.Cu") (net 8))
 (segment (start 131.9625 68.05) (end 133.0625 66.95) (width 0.25) (layer "F.Cu") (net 8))
 (segment (start 128.0625 69.95) (end 129.1625 71.05) (width 0.25) (layer "F.Cu") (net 10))
 (segment (start 129.1625 71.05) (end 133.0625 71.05) (width 0.25) (layer "F.Cu") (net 10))
 (segment (start 145.525 71.46) (end 145.525 72.73) (width 0.25) (layer "F.Cu") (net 1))
 (segment (start 151.8279 75.5801) (end 150.868 76.54) (width 0.25) (layer "F.Cu") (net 1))
 (segment (start 149.831 75.896) (end 150.475 76.54) (width 0.25) (layer "F.Cu") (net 1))
 (segment (start 146.151 75.896) (end 149.831 75.896) (width 0.25) (layer "F.Cu") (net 1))
 (segment (start 150.868 76.54) (end 150.475 76.54) (width 0.25) (layer "F.Cu") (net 1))
 (segment (start 145.525 75.27) (end 146.151 75.896) (width 0.25) (layer "F.Cu") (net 1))
 (segment (start 153.35 74) (end 151.8279 74) (width 0.25) (layer "F.Cu") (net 1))
 (segment (start 145.525 71.46) (end 150.475 71.46) (width 0.25) (layer "F.Cu") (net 1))
 (segment (start 151.8279 72.4345) (end 150.8534 71.46) (width 0.25) (layer "F.Cu") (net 1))
 (segment (start 151.8279 74) (end 150.475 74) (width 0.25) (layer "F.Cu") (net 1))
 (segment (start 151.8279 74) (end 151.8279 72.4345) (width 0.25) (layer "F.Cu") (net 1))
 (segment (start 150.8534 71.46) (end 150.475 71.46) (width 0.25) (layer "F.Cu") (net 1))
 (segment (start 151.8279 74) (end 151.8279 75.5801) (width 0.25) (layer "F.Cu") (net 1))
 (segment (start 148.7567 74) (end 150.0267 72.73) (width 0.25) (layer "F.Cu") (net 31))
 (segment (start 144.2075 73.1136) (end 145.0939 74) (width 0.25) (layer "F.Cu") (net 31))
 (segment (start 150.0267 72.73) (end 150.475 72.73) (width 0.25) (layer "F.Cu") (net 31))
 (segment (start 145.0625 64.05) (end 145.0625 64.5375) (width 0.25) (layer "F.Cu") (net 31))
 (segment (start 150.475 77.81) (end 149.831 77.166) (width 0.25) (layer "F.Cu") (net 31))
 (segment (start 145.0939 74) (end 144.2172 74.8767) (width 0.25) (layer "F.Cu") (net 31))
 (segment (start 145.0939 74) (end 145.525 74) (width 0.25) (layer "F.Cu") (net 31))
 (segment (start 145.525 74) (end 148.7567 74) (width 0.25) (layer "F.Cu") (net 31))
 (segment (start 148.7567 74) (end 150.0267 75.27) (width 0.25) (layer "F.Cu") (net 31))
 (segment (start 150.0267 75.27) (end 150.475 75.27) (width 0.25) (layer "F.Cu") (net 31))
 (segment (start 146.151 77.166) (end 145.525 76.54) (width 0.25) (layer "F.Cu") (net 31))
 (segment (start 149.831 77.166) (end 146.151 77.166) (width 0.25) (layer "F.Cu") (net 31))
 (segment (start 144.2172 75.6771) (end 145.0801 76.54) (width 0.25) (layer "F.Cu") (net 31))
 (segment (start 146.1427 66.4901) (end 144.2075 68.4253) (width 0.25) (layer "F.Cu") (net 31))
 (segment (start 144.2075 68.4253) (end 144.2075 73.1136) (width 0.25) (layer "F.Cu") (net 31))
 (segment (start 145.0625 64.5375) (end 146.1427 65.6177) (width 0.25) (layer "F.Cu") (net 31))
 (segment (start 146.1427 65.6177) (end 146.1427 66.4901) (width 0.25) (layer "F.Cu") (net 31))
 (segment (start 144.2172 74.8767) (end 144.2172 75.6771) (width 0.25) (layer "F.Cu") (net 31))
 (segment (start 145.0801 76.54) (end 145.525 76.54) (width 0.25) (layer "F.Cu") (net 31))
 (segment (start 122.95 74.35) (end 123.6003 74.35) (width 0.25) (layer "F.Cu") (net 17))
 (segment (start 123.9003 74.05) (end 127.0625 74.05) (width 0.25) (layer "F.Cu") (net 17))
 (segment (start 123.6003 74.35) (end 123.9003 74.05) (width 0.25) (layer "F.Cu") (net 17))
 (segment (start 122.95 75.65) (end 122.2997 75.65) (width 0.25) (layer "F.Cu") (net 19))
 (segment (start 122.2997 75.65) (end 122.2997 74.9494) (width 0.25) (layer "F.Cu") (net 19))
 (segment (start 122.2997 74.9494) (end 121.7003 74.35) (width 0.25) (layer "F.Cu") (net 19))
 (segment (start 121.05 74.35) (end 121.7003 74.35) (width 0.25) (layer "F.Cu") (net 19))
 (segment (start 145.4062 53.7063) (end 147.0625 52.05) (width 0.25) (layer "F.Cu") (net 23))
 (segment (start 146.8625 59.95) (end 146.4763 59.95) (width 0.25) (layer "F.Cu") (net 23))
 (segment (start 146.4763 59.95) (end 145.4062 58.8799) (width 0.25) (layer "F.Cu") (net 23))
 (segment (start 145.4062 58.8799) (end 145.4062 53.7063) (width 0.25) (layer "F.Cu") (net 23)))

